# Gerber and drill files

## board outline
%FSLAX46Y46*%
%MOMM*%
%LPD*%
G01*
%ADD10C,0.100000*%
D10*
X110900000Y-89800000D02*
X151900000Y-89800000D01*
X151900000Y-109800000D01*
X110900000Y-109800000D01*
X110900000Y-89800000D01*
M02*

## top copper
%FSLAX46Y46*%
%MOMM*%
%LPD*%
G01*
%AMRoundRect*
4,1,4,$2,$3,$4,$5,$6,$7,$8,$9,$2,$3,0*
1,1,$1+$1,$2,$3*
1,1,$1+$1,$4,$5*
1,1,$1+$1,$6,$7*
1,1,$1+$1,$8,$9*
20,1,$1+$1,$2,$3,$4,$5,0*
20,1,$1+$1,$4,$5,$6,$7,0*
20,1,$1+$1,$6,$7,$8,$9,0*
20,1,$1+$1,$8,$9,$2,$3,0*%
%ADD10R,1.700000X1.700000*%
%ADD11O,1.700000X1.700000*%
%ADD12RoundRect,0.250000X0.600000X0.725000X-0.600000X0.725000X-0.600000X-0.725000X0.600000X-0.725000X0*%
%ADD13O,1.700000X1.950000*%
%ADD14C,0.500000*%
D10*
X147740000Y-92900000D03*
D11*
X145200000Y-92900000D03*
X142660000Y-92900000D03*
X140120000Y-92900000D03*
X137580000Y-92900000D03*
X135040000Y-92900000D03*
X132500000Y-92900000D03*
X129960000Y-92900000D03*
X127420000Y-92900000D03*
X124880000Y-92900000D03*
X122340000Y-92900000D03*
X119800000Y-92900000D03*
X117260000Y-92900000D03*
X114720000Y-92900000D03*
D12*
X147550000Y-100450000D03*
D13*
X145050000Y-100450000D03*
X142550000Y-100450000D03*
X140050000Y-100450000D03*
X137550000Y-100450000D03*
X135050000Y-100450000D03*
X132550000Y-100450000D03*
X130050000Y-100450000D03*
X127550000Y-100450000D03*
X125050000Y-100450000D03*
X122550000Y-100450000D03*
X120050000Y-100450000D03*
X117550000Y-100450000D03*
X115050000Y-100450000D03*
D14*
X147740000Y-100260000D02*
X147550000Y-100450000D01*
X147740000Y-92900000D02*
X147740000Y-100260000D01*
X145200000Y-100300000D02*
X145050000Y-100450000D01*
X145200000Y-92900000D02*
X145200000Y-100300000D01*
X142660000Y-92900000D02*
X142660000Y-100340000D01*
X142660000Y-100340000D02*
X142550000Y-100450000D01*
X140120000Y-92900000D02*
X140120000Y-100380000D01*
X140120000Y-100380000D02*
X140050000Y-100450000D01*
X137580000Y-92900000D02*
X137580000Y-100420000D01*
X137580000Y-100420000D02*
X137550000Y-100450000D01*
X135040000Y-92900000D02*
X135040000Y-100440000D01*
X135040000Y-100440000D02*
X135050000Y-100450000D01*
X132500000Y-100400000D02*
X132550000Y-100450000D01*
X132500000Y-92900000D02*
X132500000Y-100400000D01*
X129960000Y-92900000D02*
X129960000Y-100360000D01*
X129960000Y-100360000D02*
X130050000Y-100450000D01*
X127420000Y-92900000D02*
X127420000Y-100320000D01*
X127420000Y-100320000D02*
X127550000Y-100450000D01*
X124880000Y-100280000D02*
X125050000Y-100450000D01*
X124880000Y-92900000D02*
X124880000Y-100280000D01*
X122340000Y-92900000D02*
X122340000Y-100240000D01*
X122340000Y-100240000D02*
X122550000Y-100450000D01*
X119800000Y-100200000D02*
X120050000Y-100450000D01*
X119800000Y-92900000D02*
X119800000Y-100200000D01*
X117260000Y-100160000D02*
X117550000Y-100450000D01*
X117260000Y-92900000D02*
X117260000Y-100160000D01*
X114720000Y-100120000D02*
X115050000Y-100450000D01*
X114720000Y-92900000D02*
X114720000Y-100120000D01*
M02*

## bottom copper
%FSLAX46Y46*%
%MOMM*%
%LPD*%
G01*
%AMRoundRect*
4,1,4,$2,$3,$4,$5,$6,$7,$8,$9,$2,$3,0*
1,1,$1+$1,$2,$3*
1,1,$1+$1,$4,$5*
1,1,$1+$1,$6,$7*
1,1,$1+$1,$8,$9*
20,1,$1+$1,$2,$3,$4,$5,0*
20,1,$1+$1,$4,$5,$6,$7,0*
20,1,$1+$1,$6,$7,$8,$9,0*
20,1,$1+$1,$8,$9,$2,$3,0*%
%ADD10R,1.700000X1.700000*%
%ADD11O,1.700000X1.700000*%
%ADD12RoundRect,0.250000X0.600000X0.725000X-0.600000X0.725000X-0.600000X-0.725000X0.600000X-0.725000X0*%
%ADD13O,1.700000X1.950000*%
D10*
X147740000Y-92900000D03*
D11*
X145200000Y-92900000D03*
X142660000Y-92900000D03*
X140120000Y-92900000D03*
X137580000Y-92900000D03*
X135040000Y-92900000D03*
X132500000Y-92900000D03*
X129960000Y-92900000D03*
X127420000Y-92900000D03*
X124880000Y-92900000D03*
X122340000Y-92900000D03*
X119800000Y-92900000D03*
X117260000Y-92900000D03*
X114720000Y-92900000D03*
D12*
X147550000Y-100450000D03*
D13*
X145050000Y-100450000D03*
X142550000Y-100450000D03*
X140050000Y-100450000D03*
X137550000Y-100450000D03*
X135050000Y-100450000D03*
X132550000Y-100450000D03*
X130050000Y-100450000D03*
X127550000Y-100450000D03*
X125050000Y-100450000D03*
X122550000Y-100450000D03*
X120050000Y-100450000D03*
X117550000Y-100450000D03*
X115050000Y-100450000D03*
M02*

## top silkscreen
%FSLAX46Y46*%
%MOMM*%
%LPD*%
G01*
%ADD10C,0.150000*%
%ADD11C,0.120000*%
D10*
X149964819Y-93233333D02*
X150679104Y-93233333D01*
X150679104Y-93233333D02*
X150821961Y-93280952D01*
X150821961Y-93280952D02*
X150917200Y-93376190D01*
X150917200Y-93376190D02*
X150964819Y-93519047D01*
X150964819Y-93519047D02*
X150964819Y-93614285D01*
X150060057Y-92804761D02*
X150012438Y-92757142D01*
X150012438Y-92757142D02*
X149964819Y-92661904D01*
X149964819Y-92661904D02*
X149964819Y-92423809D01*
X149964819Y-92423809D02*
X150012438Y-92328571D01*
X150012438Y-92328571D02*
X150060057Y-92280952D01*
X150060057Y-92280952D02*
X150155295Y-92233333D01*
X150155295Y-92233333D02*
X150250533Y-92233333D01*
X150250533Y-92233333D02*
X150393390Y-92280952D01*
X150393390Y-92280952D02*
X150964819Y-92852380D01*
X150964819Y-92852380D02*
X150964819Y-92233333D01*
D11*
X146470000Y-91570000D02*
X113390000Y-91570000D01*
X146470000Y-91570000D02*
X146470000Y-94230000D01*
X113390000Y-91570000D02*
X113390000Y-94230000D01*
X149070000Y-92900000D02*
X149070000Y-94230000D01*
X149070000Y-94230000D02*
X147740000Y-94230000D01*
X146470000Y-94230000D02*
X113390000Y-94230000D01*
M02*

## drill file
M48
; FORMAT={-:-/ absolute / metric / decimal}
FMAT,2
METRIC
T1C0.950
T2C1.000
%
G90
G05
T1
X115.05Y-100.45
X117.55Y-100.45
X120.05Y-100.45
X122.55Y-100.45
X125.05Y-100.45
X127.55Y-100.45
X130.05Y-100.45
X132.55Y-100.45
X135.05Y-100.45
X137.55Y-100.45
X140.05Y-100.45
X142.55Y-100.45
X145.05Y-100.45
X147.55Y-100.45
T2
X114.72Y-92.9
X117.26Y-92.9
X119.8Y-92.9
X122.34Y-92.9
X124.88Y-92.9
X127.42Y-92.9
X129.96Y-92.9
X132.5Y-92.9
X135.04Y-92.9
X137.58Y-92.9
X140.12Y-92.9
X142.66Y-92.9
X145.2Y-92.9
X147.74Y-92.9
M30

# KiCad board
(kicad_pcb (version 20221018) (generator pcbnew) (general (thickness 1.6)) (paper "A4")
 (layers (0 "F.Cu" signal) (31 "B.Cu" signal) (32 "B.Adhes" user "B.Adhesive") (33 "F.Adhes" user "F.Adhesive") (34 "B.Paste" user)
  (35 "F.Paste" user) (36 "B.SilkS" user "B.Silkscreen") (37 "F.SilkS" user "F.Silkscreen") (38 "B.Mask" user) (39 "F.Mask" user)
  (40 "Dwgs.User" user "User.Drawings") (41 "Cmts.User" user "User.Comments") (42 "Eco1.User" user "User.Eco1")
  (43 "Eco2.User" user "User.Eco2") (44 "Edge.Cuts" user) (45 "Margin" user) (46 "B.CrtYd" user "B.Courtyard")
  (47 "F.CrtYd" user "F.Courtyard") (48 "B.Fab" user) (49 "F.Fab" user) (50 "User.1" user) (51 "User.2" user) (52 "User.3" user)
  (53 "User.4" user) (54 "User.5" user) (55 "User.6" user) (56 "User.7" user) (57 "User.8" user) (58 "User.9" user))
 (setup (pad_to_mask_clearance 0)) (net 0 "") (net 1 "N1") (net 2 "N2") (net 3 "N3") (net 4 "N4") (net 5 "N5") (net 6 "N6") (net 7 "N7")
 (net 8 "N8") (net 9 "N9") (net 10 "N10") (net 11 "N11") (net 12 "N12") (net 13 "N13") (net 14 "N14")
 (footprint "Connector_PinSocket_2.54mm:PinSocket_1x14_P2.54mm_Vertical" (layer "F.Cu") (at 147.74 92.9 -90)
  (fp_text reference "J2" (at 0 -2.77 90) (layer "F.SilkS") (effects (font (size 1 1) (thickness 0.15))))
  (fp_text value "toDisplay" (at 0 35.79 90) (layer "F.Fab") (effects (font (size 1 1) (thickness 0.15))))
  (fp_line (start -1.33 1.27) (end -1.33 34.35) (stroke (width 0.12) (type solid)) (layer "F.SilkS"))
  (fp_line (start -1.33 1.27) (end 1.33 1.27) (stroke (width 0.12) (type solid)) (layer "F.SilkS"))
  (fp_line (start -1.33 34.35) (end 1.33 34.35) (stroke (width 0.12) (type solid)) (layer "F.SilkS"))
  (fp_line (start 0 -1.33) (end 1.33 -1.33) (stroke (width 0.12) (type solid)) (layer "F.SilkS"))
  (fp_line (start 1.33 -1.33) (end 1.33 0) (stroke (width 0.12) (type solid)) (layer "F.SilkS"))
  (fp_line (start 1.33 1.27) (end 1.33 34.35) (stroke (width 0.12) (type solid)) (layer "F.SilkS"))
  (pad "1" thru_hole rect (at 0 0 270) (size 1.7 1.7) (drill 1) (layers "*.Cu" "*.Mask") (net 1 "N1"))
  (pad "2" thru_hole oval (at 0 2.54 270) (size 1.7 1.7) (drill 1) (layers "*.Cu" "*.Mask") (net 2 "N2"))
  (pad "3" thru_hole oval (at 0 5.08 270) (size 1.7 1.7) (drill 1) (layers "*.Cu" "*.Mask") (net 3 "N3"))
  (pad "4" thru_hole oval (at 0 7.62 270) (size 1.7 1.7) (drill 1) (layers "*.Cu" "*.Mask") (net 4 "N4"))
  (pad "5" thru_hole oval (at 0 10.16 270) (size 1.7 1.7) (drill 1) (layers "*.Cu" "*.Mask") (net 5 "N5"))
  (pad "6" thru_hole oval (at 0 12.7 270) (size 1.7 1.7) (drill 1) (layers "*.Cu" "*.Mask") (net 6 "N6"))
  (pad "7" thru_hole oval (at 0 15.24 270) (size 1.7 1.7) (drill 1) (layers "*.Cu" "*.Mask") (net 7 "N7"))
  (pad "8" thru_hole oval (at 0 17.78 270) (size 1.7 1.7) (drill 1) (layers "*.Cu" "*.Mask") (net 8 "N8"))
  (pad "9" thru_hole oval (at 0 20.32 270) (size 1.7 1.7) (drill 1) (layers "*.Cu" "*.Mask") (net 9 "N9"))
  (pad "10" thru_hole oval (at 0 22.86 270) (size 1.7 1.7) (drill 1) (layers "*.Cu" "*.Mask") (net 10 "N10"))
  (pad "11" thru_hole oval (at 0 25.4 270) (size 1.7 1.7) (drill 1) (layers "*.Cu" "*.Mask") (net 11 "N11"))
  (pad "12" thru_hole oval (at 0 27.94 270) (size 1.7 1.7) (drill 1) (layers "*.Cu" "*.Mask") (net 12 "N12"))
  (pad "13" thru_hole oval (at 0 30.48 270) (size 1.7 1.7) (drill 1) (layers "*.Cu" "*.Mask") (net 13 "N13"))
  (pad "14" thru_hole oval (at 0 33.02 270) (size 1.7 1.7) (drill 1) (layers "*.Cu" "*.Mask") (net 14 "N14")))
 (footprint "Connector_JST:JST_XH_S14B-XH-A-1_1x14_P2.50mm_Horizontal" (layer "B.Cu") (at 147.55 100.45 180)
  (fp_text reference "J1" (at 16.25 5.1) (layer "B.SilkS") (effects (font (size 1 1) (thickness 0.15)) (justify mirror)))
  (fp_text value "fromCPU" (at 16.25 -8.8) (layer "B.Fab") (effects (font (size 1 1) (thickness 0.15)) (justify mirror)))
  (pad "1" thru_hole roundrect (at 0 0 180) (size 1.7 1.95) (drill 0.95) (layers "*.Cu" "*.Mask") (roundrect_rratio 0.147059) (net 1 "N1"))
  (pad "2" thru_hole oval (at 2.5 0 180) (size 1.7 1.95) (drill 0.95) (layers "*.Cu" "*.Mask") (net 2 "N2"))
  (pad "3" thru_hole oval (at 5 0 180) (size 1.7 1.95) (drill 0.95) (layers "*.Cu" "*.Mask") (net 3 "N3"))
  (pad "4" thru_hole oval (at 7.5 0 180) (size 1.7 1.95) (drill 0.95) (layers "*.Cu" "*.Mask") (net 4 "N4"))
  (pad "5" thru_hole oval (at 10 0 180) (size 1.7 1.95) (drill 0.95) (layers "*.Cu" "*.Mask") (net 5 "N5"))
  (pad "6" thru_hole oval (at 12.5 0 180) (size 1.7 1.95) (drill 0.95) (layers "*.Cu" "*.Mask") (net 6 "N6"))
  (pad "7" thru_hole oval (at 15 0 180) (size 1.7 1.95) (drill 0.95) (layers "*.Cu" "*.Mask") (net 7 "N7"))
  (pad "8" thru_hole oval (at 17.5 0 180) (size 1.7 1.95) (drill 0.95) (layers "*.Cu" "*.Mask") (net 8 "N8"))
  (pad "9" thru_hole oval (at 20 0 180) (size 1.7 1.95) (drill 0.95) (layers "*.Cu" "*.Mask") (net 9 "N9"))
  (pad "10" thru_hole oval (at 22.5 0 180) (size 1.7 1.95) (drill 0.95) (layers "*.Cu" "*.Mask") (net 10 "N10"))
  (pad "11" thru_hole oval (at 25 0 180) (size 1.7 1.95) (drill 0.95) (layers "*.Cu" "*.Mask") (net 11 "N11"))
  (pad "12" thru_hole oval (at 27.5 0 180) (size 1.7 1.95) (drill 0.95) (layers "*.Cu" "*.Mask") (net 12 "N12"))
  (pad "13" thru_hole oval (at 30 0 180) (size 1.7 1.95) (drill 0.95) (layers "*.Cu" "*.Mask") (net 13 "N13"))
  (pad "14" thru_hole oval (at 32.5 0 180) (size 1.7 1.95) (drill 0.95) (layers "*.Cu" "*.Mask") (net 14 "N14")))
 (gr_rect (start 110.9 89.8) (end 151.9 109.8) (stroke (width 0.1) (type default)) (fill none) (layer "Edge.Cuts"))
 (segment (start 147.74 100.26) (end 147.55 100.45) (width 0.5) (layer "F.Cu") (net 1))
 (segment (start 147.74 92.9) (end 147.74 100.26) (width 0.5) (layer "F.Cu") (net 1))
 (segment (start 145.2 100.3) (end 145.05 100.45) (width 0.5) (layer "F.Cu") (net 2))
 (segment (start 145.2 92.9) (end 145.2 100.3) (width 0.5) (layer "F.Cu") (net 2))
 (segment (start 142.66 92.9) (end 142.66 100.34) (width 0.5) (layer "F.Cu") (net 3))
 (segment (start 142.66 100.34) (end 142.55 100.45) (width 0.5) (layer "F.Cu") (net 3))
 (segment (start 140.12 92.9) (end 140.12 100.38) (width 0.5) (layer "F.Cu") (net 4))
 (segment (start 140.12 100.38) (end 140.05 100.45) (width 0.5) (layer "F.Cu") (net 4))
 (segment (start 137.58 92.9) (end 137.58 100.42) (width 0.5) (layer "F.Cu") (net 5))
 (segment (start 137.58 100.42) (end 137.55 100.45) (width 0.5) (layer "F.Cu") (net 5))
 (segment (start 135.04 92.9) (end 135.04 100.44) (width 0.5) (layer "F.Cu") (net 6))
 (segment (start 135.04 100.44) (end 135.05 100.45) (width 0.5) (layer "F.Cu") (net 6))
 (segment (start 132.5 100.4) (end 132.55 100.45) (width 0.5) (layer "F.Cu") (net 7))
 (segment (start 132.5 92.9) (end 132.5 100.4) (width 0.5) (layer "F.Cu") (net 7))
 (segment (start 129.96 92.9) (end 129.96 100.36) (width 0.5) (layer "F.Cu") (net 8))
 (segment (start 129.96 100.36) (end 130.05 100.45) (width 0.5) (layer "F.Cu") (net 8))
 (segment (start 127.42 92.9) (end 127.42 100.32) (width 0.5) (layer "F.Cu") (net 9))
 (segment (start 127.42 100.32) (end 127.55 100.45) (width 0.5) (layer "F.Cu") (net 9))
 (segment (start 124.88 100.28) (end 125.05 100.45) (width 0.5) (layer "F.Cu") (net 10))
 (segment (start 124.88 92.9) (end 124.88 100.28) (width 0.5) (layer "F.Cu") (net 10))
 (segment (start 122.34 92.9) (end 122.34 100.24) (width 0.5) (layer "F.Cu") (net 11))
 (segment (start 122.34 100.24) (end 122.55 100.45) (width 0.5) (layer "F.Cu") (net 11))
 (segment (start 119.8 100.2) (end 120.05 100.45) (width 0.5) (layer "F.Cu") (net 12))
 (segment (start 119.8 92.9) (end 119.8 100.2) (width 0.5) (layer "F.Cu") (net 12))
 (segment (start 117.26 100.16) (end 117.55 100.45) (width 0.5) (layer "F.Cu") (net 13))
 (segment (start 117.26 92.9) (end 117.26 100.16) (width 0.5) (layer "F.Cu") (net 13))
 (segment (start 114.72 100.12) (end 115.05 100.45) (width 0.5) (layer "F.Cu") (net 14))
 (segment (start 114.72 92.9) (end 114.72 100.12) (width 0.5) (layer "F.Cu") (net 14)))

